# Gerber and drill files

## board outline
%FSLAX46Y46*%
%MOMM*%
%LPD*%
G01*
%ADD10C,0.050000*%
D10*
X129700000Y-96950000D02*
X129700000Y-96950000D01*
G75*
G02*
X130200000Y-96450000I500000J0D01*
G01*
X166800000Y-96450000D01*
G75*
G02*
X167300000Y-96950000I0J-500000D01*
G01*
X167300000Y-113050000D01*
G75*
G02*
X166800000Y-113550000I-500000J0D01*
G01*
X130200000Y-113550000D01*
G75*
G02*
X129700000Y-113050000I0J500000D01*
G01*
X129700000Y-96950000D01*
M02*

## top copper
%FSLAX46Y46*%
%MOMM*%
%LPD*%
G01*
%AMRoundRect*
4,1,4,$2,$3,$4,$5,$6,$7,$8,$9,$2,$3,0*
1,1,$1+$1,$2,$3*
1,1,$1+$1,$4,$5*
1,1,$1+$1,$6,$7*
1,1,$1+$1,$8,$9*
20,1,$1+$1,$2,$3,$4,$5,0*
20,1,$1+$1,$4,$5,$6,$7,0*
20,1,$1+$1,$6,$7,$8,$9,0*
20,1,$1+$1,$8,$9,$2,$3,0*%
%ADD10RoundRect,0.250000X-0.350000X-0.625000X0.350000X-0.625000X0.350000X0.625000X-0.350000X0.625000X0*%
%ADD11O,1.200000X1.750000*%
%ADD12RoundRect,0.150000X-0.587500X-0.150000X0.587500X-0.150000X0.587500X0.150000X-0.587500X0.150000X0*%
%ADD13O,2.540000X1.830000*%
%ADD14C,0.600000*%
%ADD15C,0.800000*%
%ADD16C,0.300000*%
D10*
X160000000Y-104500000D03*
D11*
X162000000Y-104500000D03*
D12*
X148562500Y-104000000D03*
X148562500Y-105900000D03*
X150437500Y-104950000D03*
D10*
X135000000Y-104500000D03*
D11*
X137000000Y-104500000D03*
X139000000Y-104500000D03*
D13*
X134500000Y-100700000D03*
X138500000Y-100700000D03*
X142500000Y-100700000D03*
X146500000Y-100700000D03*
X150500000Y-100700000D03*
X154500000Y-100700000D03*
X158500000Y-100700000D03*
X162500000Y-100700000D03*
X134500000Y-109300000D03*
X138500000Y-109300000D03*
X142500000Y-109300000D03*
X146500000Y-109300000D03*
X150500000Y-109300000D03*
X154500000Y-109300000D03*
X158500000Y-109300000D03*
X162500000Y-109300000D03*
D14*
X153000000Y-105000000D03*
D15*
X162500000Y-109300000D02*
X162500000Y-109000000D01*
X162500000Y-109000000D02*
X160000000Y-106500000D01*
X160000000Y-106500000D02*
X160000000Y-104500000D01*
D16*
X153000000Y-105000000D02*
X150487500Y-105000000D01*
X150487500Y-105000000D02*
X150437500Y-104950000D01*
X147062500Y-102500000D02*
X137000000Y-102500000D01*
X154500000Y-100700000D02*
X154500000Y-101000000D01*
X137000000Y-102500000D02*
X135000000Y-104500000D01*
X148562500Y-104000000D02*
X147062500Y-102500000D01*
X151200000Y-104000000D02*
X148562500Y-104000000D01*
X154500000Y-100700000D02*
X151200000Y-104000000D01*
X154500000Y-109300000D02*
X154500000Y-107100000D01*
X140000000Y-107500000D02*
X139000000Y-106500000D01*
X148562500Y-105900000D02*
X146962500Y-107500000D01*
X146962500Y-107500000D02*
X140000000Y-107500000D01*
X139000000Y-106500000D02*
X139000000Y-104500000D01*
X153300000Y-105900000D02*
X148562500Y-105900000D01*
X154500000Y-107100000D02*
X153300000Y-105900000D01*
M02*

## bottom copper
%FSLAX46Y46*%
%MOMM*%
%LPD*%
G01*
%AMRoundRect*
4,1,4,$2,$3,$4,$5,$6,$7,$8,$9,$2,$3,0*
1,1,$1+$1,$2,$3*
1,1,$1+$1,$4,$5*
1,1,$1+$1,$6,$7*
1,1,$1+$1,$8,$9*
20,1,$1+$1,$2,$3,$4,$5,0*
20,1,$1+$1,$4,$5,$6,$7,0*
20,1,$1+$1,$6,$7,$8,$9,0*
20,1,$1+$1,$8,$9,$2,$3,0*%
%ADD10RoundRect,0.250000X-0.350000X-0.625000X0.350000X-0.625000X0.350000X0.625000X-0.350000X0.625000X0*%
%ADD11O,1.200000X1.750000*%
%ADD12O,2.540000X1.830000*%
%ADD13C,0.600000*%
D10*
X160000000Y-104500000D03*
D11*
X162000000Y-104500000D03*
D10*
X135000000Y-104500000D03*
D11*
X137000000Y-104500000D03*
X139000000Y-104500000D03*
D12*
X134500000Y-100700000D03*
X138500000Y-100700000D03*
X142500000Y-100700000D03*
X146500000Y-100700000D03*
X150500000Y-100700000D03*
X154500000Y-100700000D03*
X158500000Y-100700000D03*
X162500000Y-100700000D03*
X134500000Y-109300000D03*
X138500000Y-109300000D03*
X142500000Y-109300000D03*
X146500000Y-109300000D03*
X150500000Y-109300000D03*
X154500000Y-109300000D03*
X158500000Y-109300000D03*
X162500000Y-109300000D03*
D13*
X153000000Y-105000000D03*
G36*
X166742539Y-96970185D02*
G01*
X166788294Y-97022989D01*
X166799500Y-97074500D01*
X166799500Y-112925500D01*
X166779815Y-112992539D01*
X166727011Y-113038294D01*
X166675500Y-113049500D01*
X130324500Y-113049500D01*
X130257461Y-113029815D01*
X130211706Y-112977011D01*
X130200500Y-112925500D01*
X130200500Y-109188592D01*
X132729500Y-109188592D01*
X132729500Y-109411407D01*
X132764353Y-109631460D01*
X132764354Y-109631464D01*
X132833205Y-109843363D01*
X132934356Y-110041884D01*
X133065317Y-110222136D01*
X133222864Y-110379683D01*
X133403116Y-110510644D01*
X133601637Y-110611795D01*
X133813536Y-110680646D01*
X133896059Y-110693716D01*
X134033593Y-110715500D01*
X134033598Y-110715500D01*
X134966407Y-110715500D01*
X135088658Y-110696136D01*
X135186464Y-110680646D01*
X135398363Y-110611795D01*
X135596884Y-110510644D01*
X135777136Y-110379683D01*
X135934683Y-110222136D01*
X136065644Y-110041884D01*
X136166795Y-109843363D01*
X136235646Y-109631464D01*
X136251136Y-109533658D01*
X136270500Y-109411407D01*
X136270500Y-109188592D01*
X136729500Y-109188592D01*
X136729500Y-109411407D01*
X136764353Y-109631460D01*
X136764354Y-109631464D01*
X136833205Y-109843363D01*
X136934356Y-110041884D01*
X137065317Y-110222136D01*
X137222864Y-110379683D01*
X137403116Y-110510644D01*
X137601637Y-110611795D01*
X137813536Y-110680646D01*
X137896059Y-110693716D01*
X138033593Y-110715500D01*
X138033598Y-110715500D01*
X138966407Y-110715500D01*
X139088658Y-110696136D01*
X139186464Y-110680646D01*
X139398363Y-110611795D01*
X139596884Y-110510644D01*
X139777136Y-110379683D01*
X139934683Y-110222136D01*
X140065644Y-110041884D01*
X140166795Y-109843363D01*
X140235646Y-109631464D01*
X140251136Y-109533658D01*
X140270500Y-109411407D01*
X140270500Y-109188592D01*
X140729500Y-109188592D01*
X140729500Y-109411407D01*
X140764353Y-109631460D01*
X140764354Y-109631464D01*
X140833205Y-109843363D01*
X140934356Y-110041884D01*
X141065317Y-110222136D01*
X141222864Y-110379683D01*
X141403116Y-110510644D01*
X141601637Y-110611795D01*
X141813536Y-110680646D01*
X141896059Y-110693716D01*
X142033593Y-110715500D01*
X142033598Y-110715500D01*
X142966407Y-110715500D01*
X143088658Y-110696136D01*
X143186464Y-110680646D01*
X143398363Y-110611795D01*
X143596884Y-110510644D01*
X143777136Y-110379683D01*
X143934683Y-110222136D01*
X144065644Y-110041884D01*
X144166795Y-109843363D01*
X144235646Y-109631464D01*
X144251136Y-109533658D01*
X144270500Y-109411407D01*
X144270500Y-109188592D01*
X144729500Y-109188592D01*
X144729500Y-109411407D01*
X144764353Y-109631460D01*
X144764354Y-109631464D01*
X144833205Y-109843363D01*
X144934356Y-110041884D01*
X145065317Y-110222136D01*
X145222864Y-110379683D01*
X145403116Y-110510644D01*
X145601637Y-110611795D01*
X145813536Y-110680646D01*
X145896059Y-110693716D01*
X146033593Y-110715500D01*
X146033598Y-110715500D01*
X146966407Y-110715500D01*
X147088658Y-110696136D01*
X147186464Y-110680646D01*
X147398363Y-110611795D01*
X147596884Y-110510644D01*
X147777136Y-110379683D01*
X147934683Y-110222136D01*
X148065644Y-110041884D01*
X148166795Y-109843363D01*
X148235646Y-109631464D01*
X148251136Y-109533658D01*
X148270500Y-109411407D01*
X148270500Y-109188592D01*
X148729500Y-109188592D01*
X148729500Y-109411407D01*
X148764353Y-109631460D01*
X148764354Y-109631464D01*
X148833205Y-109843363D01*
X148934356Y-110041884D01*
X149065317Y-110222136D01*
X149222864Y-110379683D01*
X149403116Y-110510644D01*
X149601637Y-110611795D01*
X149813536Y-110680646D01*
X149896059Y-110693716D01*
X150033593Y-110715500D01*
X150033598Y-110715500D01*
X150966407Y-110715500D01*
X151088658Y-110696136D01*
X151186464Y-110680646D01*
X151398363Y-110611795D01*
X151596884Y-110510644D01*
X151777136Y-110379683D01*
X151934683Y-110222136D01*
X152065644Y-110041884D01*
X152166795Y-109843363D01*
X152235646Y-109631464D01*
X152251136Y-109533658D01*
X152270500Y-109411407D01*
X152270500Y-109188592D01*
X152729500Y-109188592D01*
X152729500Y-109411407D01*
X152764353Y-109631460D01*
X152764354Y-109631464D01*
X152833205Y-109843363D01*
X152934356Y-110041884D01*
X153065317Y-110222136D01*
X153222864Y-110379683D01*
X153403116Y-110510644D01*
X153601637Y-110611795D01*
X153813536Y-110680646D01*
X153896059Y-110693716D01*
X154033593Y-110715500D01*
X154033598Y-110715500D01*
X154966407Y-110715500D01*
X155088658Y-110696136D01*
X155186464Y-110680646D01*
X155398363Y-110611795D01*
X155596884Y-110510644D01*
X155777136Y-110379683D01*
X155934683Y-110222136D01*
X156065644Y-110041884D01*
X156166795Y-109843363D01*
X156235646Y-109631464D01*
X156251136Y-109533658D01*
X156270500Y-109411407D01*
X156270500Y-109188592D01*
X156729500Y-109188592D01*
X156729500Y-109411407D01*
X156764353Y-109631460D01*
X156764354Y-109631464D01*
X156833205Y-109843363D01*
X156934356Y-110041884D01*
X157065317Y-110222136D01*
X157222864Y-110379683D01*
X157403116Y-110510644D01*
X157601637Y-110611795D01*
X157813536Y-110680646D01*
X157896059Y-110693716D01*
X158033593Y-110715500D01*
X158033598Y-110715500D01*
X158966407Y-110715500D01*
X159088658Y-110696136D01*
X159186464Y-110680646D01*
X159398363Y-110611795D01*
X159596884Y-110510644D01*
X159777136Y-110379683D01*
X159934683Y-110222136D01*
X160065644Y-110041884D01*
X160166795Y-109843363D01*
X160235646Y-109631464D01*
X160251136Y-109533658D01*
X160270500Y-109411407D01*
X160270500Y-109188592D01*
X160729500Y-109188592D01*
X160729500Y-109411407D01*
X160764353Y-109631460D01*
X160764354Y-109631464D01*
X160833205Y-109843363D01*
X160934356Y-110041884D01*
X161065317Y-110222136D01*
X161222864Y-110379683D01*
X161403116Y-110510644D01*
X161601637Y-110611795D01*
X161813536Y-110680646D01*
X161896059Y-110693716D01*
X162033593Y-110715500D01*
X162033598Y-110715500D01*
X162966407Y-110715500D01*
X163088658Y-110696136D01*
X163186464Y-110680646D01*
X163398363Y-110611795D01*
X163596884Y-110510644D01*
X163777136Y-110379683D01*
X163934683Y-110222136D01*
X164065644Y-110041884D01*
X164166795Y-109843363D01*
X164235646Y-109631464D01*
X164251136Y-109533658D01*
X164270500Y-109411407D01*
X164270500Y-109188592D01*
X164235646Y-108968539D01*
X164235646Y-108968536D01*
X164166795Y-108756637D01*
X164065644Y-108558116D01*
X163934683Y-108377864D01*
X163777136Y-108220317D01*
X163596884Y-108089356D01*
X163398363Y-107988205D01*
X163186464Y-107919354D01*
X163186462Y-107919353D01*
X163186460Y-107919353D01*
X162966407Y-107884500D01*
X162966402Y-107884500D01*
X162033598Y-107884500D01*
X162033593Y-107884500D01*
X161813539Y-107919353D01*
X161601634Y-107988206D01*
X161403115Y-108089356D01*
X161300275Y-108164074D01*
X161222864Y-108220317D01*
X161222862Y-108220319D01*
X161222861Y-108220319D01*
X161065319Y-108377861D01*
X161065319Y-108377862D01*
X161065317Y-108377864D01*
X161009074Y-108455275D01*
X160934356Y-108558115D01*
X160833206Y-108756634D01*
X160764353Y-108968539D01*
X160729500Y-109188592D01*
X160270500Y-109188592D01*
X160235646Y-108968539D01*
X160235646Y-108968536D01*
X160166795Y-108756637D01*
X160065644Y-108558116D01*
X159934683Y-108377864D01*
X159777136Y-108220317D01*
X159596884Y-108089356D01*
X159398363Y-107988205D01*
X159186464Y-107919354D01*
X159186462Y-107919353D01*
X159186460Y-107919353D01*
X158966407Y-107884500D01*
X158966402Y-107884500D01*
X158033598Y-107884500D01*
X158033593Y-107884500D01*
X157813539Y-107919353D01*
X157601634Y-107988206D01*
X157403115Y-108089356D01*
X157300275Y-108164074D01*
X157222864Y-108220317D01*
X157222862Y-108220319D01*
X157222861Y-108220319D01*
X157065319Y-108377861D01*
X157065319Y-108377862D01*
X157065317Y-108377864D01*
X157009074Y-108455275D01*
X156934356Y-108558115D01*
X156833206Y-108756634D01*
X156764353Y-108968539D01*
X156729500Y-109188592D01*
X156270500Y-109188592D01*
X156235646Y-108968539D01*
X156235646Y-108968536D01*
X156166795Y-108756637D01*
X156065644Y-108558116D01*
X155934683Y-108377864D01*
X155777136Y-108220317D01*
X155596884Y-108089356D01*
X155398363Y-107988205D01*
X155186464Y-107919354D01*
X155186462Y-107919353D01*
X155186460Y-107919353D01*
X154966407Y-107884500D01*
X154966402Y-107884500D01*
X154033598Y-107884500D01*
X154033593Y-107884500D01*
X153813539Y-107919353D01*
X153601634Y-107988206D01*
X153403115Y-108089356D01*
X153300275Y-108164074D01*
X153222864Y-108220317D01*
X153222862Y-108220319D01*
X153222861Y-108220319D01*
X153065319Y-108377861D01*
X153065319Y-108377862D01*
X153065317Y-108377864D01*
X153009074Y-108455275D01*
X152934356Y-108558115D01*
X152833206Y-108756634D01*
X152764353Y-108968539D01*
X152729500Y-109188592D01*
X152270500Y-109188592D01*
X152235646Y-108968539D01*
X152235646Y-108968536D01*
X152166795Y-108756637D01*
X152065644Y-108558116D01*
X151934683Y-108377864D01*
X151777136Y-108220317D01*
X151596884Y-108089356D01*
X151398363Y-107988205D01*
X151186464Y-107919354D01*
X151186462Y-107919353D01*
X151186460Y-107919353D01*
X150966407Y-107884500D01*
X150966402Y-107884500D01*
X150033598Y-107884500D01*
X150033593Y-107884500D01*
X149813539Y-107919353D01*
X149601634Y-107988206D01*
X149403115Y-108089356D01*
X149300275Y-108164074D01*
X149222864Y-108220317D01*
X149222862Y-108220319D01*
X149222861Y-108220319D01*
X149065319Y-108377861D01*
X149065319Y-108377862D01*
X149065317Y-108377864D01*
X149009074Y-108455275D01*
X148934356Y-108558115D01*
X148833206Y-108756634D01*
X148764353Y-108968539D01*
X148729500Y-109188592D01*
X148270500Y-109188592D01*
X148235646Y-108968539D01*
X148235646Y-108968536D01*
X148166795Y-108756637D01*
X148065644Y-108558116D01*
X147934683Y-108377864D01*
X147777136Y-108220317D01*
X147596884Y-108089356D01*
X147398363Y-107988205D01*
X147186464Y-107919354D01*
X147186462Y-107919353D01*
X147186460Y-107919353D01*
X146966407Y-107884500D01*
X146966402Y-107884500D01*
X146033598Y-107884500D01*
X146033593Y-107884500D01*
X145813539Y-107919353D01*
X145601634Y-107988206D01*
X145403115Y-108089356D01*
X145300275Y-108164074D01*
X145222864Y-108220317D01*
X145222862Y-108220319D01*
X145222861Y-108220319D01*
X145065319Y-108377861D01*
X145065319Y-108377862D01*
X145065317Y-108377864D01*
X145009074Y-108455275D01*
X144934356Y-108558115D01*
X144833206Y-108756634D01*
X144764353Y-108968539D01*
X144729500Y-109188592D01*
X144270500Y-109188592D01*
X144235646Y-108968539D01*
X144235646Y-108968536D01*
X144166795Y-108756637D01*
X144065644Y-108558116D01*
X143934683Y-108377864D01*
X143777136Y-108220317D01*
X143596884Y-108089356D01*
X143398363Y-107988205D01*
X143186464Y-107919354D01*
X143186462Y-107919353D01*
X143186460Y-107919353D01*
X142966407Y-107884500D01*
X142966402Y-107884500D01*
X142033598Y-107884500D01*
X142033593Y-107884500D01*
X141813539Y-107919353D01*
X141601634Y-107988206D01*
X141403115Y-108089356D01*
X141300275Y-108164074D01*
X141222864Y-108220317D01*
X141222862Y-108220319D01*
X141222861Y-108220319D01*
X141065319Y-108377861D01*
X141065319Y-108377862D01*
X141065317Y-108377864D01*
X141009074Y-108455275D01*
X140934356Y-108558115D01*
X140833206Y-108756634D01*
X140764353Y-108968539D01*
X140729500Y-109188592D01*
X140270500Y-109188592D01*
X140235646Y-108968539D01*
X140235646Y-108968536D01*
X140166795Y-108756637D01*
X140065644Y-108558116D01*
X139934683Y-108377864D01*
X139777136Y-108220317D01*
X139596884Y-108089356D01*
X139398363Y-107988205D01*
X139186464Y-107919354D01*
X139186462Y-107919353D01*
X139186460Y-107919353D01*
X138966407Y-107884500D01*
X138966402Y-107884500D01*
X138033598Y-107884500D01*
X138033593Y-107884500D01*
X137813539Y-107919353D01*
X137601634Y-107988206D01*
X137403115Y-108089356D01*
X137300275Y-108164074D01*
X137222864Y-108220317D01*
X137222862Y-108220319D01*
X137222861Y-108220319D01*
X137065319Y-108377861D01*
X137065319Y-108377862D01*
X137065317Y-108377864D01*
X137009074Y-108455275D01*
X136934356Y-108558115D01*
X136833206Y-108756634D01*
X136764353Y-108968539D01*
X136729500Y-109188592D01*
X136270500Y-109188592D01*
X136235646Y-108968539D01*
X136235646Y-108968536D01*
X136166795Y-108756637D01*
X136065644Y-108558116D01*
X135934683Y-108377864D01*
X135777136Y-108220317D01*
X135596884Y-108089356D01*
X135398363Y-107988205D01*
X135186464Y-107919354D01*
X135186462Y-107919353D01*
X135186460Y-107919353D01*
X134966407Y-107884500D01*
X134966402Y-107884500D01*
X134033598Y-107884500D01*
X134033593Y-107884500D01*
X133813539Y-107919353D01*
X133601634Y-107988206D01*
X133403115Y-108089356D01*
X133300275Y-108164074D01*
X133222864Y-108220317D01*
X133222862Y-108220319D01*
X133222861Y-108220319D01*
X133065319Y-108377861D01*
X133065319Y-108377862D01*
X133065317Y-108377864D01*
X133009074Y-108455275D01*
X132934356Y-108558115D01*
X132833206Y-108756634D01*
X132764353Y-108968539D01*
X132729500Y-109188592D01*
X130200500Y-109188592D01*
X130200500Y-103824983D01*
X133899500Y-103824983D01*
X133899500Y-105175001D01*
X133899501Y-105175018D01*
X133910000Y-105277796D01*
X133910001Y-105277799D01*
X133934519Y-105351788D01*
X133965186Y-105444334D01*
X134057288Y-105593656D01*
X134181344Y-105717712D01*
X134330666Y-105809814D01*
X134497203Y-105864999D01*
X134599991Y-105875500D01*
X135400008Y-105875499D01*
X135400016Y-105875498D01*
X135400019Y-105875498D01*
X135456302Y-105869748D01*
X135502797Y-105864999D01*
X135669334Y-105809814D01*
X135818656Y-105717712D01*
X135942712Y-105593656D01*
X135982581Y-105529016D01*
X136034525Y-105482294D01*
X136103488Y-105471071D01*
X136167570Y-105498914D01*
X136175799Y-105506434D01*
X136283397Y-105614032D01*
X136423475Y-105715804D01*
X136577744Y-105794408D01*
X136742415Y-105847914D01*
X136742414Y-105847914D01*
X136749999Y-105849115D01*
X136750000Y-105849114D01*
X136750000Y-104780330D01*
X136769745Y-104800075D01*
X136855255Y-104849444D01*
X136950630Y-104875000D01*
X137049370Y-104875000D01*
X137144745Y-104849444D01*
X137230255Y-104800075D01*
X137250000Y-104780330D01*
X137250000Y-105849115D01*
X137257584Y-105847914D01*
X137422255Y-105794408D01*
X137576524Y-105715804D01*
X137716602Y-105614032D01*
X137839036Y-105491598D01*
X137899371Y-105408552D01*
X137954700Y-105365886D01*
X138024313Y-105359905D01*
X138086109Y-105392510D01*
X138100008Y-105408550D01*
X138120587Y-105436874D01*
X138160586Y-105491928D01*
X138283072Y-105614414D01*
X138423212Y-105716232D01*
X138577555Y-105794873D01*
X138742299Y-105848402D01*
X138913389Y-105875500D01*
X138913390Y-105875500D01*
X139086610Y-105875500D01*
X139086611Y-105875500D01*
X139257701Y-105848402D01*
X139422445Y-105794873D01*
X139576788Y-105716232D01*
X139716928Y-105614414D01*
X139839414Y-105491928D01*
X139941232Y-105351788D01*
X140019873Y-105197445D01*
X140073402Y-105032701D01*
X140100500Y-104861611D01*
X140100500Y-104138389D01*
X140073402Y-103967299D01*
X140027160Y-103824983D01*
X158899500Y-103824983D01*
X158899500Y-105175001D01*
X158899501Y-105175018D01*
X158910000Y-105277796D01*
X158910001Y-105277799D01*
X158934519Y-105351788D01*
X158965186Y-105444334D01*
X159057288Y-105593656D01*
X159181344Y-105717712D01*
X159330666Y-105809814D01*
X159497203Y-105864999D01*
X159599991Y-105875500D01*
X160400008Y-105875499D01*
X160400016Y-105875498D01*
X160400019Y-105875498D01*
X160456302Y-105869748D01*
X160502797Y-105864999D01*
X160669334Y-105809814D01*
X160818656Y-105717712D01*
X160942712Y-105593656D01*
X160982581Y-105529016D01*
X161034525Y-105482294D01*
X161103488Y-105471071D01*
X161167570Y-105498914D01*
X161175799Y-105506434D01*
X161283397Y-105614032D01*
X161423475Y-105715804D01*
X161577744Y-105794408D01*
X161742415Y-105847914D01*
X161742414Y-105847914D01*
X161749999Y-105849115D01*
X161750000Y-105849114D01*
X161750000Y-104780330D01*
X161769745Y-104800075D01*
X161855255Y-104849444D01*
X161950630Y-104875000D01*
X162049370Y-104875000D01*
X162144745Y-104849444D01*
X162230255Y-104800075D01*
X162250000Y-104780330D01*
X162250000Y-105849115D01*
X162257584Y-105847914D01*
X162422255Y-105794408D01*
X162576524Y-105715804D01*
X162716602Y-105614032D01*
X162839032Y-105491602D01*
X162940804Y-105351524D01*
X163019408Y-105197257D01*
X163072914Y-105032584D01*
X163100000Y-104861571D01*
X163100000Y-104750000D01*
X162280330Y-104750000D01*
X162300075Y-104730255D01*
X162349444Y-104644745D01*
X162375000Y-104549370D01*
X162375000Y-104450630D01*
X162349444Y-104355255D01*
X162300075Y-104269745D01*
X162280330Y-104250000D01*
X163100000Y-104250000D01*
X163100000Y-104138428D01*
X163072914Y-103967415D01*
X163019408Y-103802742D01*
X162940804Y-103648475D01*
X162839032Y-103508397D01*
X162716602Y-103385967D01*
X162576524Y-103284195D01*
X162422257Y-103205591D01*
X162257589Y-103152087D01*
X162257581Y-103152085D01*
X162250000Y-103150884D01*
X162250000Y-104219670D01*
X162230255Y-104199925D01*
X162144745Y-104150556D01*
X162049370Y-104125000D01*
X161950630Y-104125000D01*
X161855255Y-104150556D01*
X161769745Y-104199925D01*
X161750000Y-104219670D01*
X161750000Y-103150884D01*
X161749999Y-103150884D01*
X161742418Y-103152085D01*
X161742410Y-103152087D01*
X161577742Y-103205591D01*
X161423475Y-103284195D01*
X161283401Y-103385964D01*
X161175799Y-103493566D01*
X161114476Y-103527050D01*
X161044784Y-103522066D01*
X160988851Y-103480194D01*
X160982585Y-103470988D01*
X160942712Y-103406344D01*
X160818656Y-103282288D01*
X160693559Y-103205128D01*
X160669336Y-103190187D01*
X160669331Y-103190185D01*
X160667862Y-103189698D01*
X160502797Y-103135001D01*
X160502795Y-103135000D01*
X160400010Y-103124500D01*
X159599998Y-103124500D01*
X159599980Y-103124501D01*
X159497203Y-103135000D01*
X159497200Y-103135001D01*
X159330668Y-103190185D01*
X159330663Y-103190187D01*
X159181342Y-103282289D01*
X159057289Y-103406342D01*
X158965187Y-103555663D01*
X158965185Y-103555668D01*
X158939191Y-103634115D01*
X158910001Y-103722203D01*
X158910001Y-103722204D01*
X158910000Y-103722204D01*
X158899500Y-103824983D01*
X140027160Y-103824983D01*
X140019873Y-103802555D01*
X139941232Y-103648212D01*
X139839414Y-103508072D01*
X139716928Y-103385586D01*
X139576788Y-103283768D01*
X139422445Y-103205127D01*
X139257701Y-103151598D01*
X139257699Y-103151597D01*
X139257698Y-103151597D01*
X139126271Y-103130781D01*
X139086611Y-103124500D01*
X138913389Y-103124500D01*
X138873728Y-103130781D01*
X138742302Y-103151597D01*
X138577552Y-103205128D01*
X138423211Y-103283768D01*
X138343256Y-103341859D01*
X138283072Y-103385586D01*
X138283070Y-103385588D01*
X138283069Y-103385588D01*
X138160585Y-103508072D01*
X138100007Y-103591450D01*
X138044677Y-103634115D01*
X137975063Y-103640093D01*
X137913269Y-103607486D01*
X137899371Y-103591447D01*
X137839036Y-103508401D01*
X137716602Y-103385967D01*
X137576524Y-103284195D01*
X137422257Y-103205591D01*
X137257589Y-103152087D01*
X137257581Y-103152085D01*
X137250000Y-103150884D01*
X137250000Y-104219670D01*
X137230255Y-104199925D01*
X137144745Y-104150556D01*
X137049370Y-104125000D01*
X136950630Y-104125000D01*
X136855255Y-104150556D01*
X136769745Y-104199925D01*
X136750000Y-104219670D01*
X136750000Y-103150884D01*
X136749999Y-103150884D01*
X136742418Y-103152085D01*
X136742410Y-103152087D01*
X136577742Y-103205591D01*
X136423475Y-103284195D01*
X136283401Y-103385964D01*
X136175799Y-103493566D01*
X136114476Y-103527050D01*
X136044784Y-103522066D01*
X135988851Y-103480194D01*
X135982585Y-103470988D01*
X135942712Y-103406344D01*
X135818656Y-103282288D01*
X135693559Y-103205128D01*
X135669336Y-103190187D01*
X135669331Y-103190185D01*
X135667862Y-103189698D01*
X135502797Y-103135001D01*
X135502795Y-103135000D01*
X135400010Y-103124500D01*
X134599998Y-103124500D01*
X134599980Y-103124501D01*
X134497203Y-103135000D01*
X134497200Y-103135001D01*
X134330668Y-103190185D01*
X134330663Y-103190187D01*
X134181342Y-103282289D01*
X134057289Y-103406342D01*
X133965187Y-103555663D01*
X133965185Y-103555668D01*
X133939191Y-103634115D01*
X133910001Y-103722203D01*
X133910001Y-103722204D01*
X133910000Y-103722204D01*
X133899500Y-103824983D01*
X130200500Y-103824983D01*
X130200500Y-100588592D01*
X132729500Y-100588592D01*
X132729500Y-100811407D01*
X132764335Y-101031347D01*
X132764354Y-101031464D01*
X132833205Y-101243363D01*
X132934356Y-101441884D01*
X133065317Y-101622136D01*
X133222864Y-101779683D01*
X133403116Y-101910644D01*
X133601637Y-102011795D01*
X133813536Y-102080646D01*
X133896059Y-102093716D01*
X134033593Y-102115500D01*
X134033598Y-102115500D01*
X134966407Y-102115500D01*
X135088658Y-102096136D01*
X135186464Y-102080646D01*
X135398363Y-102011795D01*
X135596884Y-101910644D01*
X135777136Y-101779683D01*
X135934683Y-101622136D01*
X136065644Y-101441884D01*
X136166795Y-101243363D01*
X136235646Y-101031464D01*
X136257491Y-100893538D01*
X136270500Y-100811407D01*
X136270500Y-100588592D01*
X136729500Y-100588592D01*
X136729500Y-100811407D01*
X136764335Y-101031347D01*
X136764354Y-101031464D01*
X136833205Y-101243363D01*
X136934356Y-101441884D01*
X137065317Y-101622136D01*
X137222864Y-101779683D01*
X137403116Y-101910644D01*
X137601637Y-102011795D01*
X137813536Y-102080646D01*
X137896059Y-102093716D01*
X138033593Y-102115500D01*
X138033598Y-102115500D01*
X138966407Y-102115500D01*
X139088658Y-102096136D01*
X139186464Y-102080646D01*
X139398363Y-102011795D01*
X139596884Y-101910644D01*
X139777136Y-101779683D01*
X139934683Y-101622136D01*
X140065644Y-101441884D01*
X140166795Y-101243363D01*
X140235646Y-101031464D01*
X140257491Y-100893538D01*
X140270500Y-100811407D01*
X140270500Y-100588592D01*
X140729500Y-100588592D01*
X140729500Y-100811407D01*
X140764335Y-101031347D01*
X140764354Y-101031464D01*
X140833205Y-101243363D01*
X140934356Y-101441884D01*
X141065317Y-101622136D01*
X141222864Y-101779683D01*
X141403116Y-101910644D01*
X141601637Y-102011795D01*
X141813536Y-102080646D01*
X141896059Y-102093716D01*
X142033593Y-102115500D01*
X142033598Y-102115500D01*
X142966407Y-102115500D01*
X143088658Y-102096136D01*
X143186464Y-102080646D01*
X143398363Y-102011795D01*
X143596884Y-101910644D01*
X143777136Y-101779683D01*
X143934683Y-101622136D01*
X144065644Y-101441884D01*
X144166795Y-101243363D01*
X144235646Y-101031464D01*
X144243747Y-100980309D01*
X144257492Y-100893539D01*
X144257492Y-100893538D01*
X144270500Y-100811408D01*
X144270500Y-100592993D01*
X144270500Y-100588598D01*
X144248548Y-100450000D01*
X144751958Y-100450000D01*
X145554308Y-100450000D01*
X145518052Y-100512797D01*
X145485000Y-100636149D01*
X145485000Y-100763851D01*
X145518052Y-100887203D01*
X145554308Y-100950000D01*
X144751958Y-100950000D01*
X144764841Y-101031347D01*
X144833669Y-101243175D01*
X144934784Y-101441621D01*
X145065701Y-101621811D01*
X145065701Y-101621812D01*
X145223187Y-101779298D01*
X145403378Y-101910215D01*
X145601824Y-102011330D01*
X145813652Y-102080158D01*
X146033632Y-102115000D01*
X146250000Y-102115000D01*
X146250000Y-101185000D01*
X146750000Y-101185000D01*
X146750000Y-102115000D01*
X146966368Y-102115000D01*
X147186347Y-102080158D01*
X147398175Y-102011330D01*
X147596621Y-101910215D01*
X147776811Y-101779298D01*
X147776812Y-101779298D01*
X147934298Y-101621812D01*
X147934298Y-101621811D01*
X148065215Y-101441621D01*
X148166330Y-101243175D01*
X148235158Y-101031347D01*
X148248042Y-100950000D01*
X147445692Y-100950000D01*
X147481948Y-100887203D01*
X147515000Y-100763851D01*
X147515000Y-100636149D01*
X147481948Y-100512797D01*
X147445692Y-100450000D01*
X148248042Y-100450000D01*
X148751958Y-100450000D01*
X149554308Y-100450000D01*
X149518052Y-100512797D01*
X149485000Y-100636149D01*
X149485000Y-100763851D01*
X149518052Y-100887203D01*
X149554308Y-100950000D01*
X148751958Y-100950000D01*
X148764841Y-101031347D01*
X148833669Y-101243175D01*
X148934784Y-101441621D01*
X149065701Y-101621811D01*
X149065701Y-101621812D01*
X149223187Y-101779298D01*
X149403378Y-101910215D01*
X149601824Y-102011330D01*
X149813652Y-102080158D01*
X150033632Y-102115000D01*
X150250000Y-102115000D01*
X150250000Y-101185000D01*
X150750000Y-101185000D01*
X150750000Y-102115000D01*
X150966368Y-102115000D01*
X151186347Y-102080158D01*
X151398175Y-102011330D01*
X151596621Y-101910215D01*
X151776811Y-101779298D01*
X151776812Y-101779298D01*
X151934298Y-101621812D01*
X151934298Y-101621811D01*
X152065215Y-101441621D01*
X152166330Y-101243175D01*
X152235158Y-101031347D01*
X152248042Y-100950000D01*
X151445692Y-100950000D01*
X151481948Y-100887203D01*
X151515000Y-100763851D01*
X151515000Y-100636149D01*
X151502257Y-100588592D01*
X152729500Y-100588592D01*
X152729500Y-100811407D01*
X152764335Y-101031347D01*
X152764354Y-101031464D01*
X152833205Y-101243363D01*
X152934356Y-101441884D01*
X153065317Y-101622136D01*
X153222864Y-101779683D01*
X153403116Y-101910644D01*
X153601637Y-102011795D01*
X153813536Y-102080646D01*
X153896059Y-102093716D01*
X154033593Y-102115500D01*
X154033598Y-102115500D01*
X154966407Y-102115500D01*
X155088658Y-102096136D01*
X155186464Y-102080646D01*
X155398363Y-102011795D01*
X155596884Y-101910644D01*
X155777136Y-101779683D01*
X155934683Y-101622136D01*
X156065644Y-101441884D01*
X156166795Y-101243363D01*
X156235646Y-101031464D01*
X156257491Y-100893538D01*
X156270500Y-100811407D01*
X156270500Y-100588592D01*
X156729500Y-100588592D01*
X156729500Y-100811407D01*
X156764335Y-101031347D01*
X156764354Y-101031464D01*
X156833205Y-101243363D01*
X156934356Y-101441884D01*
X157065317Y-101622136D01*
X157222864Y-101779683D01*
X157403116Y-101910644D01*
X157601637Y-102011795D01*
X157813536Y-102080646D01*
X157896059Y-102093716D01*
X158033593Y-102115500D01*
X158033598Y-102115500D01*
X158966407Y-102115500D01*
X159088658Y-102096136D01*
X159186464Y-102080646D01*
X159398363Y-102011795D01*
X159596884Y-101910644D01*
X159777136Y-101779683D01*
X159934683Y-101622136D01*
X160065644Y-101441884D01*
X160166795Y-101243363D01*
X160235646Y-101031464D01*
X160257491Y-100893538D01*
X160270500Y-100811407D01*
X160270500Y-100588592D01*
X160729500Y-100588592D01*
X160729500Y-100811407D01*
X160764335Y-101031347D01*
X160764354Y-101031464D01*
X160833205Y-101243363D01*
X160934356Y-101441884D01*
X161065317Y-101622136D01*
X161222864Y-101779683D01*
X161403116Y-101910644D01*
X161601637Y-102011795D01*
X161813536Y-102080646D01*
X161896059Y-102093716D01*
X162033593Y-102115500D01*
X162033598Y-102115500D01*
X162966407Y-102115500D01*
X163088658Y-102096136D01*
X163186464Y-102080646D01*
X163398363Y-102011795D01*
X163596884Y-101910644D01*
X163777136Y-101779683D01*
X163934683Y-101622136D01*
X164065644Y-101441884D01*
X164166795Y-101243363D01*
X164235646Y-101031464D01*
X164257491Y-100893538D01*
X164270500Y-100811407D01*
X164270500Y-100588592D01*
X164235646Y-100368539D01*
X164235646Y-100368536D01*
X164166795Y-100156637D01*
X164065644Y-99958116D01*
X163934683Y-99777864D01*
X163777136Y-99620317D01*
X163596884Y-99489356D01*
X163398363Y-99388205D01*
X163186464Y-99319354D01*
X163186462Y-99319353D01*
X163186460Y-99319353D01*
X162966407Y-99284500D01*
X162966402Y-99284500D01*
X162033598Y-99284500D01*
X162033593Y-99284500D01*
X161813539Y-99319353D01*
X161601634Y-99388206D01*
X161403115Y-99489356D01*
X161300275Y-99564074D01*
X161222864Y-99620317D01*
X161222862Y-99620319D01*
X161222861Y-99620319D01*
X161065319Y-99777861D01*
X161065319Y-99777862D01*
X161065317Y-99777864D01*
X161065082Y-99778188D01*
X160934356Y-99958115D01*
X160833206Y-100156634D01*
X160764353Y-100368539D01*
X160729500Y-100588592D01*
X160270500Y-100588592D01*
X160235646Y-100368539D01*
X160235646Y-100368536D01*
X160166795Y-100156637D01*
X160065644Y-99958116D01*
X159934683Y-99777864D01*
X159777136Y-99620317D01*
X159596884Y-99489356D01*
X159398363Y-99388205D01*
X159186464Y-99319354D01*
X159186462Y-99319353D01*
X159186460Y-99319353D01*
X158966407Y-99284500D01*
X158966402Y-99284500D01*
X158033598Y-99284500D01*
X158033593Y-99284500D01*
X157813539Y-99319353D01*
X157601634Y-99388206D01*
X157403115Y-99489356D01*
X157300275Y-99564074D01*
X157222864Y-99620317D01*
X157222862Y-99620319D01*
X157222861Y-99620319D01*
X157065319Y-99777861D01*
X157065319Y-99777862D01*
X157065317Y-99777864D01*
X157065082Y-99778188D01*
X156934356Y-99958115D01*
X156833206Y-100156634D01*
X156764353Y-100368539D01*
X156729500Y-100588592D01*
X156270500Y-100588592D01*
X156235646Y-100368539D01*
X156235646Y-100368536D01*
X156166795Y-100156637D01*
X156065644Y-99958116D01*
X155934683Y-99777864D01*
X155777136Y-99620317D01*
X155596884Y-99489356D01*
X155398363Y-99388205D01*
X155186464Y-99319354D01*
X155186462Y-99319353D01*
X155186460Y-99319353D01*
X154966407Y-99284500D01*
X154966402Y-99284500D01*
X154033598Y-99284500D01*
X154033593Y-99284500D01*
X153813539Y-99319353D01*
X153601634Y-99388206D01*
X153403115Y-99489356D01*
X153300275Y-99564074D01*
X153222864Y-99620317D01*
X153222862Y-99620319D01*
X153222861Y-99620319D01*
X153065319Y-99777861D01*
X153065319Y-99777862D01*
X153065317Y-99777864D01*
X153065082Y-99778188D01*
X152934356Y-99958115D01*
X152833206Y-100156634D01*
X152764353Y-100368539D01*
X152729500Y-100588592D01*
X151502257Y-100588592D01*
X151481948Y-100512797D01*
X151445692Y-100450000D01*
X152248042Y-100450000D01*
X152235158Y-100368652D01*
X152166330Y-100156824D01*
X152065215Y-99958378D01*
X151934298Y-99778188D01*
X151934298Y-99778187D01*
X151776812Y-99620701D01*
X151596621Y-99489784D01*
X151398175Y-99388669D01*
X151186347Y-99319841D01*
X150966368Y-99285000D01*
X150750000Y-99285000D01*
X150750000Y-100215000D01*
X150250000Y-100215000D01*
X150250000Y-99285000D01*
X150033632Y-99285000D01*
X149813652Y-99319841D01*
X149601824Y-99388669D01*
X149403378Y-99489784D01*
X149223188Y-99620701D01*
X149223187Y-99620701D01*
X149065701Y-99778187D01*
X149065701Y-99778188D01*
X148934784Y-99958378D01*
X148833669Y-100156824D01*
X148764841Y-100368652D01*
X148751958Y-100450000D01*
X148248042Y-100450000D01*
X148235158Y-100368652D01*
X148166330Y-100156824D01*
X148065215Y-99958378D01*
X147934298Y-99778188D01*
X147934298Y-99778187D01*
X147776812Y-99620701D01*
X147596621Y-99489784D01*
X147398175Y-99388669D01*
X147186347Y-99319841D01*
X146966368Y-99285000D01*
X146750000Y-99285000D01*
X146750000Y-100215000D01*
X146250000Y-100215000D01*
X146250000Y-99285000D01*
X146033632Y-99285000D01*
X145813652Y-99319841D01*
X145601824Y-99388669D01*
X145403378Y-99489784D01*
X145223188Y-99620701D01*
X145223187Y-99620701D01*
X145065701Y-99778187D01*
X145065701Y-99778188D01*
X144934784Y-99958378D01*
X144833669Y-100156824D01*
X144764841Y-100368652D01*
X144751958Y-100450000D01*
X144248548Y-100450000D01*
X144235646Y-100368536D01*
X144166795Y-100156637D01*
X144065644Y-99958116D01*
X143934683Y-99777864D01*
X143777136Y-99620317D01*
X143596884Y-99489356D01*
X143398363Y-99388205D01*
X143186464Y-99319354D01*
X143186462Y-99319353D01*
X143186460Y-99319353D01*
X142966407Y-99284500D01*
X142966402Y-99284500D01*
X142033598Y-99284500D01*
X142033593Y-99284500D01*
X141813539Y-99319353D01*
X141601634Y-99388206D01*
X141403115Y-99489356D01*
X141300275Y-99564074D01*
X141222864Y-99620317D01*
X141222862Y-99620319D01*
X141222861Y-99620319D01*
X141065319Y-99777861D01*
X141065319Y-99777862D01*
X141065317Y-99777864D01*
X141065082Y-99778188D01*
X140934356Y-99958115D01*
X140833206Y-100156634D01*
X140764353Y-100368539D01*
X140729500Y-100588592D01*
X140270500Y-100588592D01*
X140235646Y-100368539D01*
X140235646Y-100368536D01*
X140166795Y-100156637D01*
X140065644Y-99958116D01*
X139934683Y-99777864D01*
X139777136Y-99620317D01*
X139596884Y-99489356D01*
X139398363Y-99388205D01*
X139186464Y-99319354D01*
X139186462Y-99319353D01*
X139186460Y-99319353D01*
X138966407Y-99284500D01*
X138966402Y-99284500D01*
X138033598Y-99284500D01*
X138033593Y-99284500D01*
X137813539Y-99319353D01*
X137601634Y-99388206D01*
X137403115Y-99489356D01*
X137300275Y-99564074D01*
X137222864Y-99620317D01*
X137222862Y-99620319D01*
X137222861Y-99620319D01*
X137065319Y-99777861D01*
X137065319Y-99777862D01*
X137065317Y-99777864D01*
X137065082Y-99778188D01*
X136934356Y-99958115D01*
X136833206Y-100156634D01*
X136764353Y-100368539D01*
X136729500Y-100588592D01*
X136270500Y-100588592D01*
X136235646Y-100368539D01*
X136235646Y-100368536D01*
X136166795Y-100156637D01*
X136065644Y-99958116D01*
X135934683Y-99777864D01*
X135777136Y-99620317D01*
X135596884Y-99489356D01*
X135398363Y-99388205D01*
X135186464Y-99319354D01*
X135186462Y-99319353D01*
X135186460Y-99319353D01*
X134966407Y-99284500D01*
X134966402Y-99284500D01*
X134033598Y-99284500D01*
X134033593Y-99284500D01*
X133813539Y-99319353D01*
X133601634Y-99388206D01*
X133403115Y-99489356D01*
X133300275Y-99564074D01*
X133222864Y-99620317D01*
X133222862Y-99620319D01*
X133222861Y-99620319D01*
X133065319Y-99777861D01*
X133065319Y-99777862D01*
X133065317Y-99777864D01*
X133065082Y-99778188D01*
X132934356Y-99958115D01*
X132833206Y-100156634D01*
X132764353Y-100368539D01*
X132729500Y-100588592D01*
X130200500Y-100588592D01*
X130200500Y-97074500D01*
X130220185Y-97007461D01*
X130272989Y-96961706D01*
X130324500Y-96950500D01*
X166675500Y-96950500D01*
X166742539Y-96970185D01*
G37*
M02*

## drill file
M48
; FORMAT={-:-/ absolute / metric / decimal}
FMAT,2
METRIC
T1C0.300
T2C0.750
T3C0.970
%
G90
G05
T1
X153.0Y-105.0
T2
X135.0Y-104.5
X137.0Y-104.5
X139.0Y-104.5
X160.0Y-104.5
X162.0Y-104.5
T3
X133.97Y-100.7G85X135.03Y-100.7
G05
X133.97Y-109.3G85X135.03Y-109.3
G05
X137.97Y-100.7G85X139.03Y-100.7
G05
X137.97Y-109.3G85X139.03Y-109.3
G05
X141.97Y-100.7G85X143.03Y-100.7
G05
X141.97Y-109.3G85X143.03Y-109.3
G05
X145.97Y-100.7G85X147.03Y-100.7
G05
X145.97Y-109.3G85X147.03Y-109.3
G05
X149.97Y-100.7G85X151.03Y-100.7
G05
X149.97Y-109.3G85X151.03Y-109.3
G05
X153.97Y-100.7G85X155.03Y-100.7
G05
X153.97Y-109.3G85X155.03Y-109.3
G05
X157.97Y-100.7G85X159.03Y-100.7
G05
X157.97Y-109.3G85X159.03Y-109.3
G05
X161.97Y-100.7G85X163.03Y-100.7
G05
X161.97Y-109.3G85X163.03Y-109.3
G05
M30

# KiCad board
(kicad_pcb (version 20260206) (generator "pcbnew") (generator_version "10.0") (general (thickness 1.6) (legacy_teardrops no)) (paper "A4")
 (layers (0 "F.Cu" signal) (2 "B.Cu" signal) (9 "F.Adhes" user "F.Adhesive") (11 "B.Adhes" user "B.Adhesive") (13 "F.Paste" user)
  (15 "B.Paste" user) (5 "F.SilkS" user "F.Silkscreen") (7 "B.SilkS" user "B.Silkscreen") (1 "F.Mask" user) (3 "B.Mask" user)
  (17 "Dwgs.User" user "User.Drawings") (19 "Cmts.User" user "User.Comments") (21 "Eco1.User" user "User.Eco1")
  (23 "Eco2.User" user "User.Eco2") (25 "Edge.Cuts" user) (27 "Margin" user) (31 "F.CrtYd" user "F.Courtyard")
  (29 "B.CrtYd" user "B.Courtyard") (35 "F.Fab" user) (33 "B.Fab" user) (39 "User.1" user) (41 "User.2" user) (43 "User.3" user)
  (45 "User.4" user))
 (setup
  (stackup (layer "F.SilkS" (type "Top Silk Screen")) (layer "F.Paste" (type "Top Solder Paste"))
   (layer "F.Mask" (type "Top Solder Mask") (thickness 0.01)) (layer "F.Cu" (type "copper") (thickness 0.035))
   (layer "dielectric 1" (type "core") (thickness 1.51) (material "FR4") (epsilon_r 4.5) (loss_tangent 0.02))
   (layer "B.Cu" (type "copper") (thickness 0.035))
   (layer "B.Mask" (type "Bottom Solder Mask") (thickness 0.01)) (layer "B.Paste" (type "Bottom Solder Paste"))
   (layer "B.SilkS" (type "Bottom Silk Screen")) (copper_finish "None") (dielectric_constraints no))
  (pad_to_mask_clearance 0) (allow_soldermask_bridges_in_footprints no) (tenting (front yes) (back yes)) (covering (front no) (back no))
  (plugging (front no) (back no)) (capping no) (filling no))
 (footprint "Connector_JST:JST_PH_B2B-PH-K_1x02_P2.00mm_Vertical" (layer "F.Cu") (at 160 104.5)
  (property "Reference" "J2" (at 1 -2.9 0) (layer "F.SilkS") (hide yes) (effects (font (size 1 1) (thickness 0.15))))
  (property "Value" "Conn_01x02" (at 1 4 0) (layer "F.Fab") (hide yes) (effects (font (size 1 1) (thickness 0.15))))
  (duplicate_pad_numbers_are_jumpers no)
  (pad "1" thru_hole roundrect (at 0 0) (size 1.2 1.75) (drill 0.75) (layers "*.Cu" "*.Mask") (remove_unused_layers no)
   (roundrect_rratio 0.208333) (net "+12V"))
  (pad "2" thru_hole oval (at 2 0) (size 1.2 1.75) (drill 0.75) (layers "*.Cu" "*.Mask") (remove_unused_layers no) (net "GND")))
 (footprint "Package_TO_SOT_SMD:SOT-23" (layer "F.Cu") (at 149.5 104.95)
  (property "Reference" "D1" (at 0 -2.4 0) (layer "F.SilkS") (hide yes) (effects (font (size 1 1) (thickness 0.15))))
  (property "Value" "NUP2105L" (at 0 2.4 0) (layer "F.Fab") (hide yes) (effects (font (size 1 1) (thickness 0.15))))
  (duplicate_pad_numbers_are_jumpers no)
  (pad "1" smd roundrect (at -0.9375 -0.95) (size 1.475 0.6) (layers "F.Cu" "F.Mask" "F.Paste") (roundrect_rratio 0.25) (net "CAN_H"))
  (pad "2" smd roundrect (at -0.9375 0.95) (size 1.475 0.6) (layers "F.Cu" "F.Mask" "F.Paste") (roundrect_rratio 0.25) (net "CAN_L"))
  (pad "3" smd roundrect (at 0.9375 0) (size 1.475 0.6) (layers "F.Cu" "F.Mask" "F.Paste") (roundrect_rratio 0.25) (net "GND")))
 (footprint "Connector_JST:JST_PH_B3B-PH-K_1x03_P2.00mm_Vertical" (layer "F.Cu") (at 135 104.5)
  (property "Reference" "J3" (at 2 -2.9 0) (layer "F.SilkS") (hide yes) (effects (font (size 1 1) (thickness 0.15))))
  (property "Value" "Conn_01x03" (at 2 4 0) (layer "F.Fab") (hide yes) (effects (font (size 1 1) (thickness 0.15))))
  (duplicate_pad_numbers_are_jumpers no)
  (pad "1" thru_hole roundrect (at 0 0) (size 1.2 1.75) (drill 0.75) (layers "*.Cu" "*.Mask") (remove_unused_layers no)
   (roundrect_rratio 0.208333) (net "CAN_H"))
  (pad "2" thru_hole oval (at 2 0) (size 1.2 1.75) (drill 0.75) (layers "*.Cu" "*.Mask") (remove_unused_layers no) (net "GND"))
  (pad "3" thru_hole oval (at 4 0) (size 1.2 1.75) (drill 0.75) (layers "*.Cu" "*.Mask") (remove_unused_layers no) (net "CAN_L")))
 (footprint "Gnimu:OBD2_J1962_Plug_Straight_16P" (layer "F.Cu") (at 148.5 105)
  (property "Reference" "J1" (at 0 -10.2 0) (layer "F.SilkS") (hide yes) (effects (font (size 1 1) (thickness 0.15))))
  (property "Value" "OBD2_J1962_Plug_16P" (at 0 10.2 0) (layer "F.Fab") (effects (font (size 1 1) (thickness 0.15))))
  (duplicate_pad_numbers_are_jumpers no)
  (pad "1" thru_hole oval (at -14 -4.3) (size 2.54 1.83) (drill oval 2.03 0.97) (layers "*.Cu" "*.Mask") (remove_unused_layers no)
   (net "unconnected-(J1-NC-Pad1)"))
  (pad "2" thru_hole oval (at -10 -4.3) (size 2.54 1.83) (drill oval 2.03 0.97) (layers "*.Cu" "*.Mask") (remove_unused_layers no)
   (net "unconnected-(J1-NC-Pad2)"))
  (pad "3" thru_hole oval (at -6 -4.3) (size 2.54 1.83) (drill oval 2.03 0.97) (layers "*.Cu" "*.Mask") (remove_unused_layers no)
   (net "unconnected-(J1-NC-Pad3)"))
  (pad "4" thru_hole oval (at -2 -4.3) (size 2.54 1.83) (drill oval 2.03 0.97) (layers "*.Cu" "*.Mask") (remove_unused_layers no)
   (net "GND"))
  (pad "5" thru_hole oval (at 2 -4.3) (size 2.54 1.83) (drill oval 2.03 0.97) (layers "*.Cu" "*.Mask") (remove_unused_layers no) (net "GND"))
  (pad "6" thru_hole oval (at 6 -4.3) (size 2.54 1.83) (drill oval 2.03 0.97) (layers "*.Cu" "*.Mask") (remove_unused_layers no)
   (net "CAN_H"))
  (pad "7" thru_hole oval (at 10 -4.3) (size 2.54 1.83) (drill oval 2.03 0.97) (layers "*.Cu" "*.Mask") (remove_unused_layers no)
   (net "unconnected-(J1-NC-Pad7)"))
  (pad "8" thru_hole oval (at 14 -4.3) (size 2.54 1.83) (drill oval 2.03 0.97) (layers "*.Cu" "*.Mask") (remove_unused_layers no)
   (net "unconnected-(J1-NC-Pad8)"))
  (pad "9" thru_hole oval (at -14 4.3) (size 2.54 1.83) (drill oval 2.03 0.97) (layers "*.Cu" "*.Mask") (remove_unused_layers no)
   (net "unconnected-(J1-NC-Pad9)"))
  (pad "10" thru_hole oval (at -10 4.3) (size 2.54 1.83) (drill oval 2.03 0.97) (layers "*.Cu" "*.Mask") (remove_unused_layers no)
   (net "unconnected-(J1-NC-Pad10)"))
  (pad "11" thru_hole oval (at -6 4.3) (size 2.54 1.83) (drill oval 2.03 0.97) (layers "*.Cu" "*.Mask") (remove_unused_layers no)
   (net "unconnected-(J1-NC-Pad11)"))
  (pad "12" thru_hole oval (at -2 4.3) (size 2.54 1.83) (drill oval 2.03 0.97) (layers "*.Cu" "*.Mask") (remove_unused_layers no)
   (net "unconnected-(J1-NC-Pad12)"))
  (pad "13" thru_hole oval (at 2 4.3) (size 2.54 1.83) (drill oval 2.03 0.97) (layers "*.Cu" "*.Mask") (remove_unused_layers no)
   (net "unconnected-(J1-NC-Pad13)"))
  (pad "14" thru_hole oval (at 6 4.3) (size 2.54 1.83) (drill oval 2.03 0.97) (layers "*.Cu" "*.Mask") (remove_unused_layers no)
   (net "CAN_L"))
  (pad "15" thru_hole oval (at 10 4.3) (size 2.54 1.83) (drill oval 2.03 0.97) (layers "*.Cu" "*.Mask") (remove_unused_layers no)
   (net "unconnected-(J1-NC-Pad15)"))
  (pad "16" thru_hole oval (at 14 4.3) (size 2.54 1.83) (drill oval 2.03 0.97) (layers "*.Cu" "*.Mask") (remove_unused_layers no)
   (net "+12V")))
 (gr_rect (start 129.7 96.45) (end 167.3 113.55) (radius 0.5) (stroke (width 0.05) (type solid)) (fill no) (locked yes) (layer "Edge.Cuts"))
 (segment (start 162.5 109.3) (end 162.5 109) (width 0.8) (layer "F.Cu") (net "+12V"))
 (segment (start 162.5 109) (end 160 106.5) (width 0.8) (layer "F.Cu") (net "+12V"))
 (segment (start 160 106.5) (end 160 104.5) (width 0.8) (layer "F.Cu") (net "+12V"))
 (segment (start 153 105) (end 150.4875 105) (width 0.3) (layer "F.Cu") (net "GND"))
 (segment (start 150.4875 105) (end 150.4375 104.95) (width 0.3) (layer "F.Cu") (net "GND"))
 (via (at 153 105) (size 0.6) (drill 0.3) (layers "F.Cu" "B.Cu") (free yes) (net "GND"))
 (segment (start 147.0625 102.5) (end 137 102.5) (width 0.3) (layer "F.Cu") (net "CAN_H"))
 (segment (start 154.5 100.7) (end 154.5 101) (width 0.3) (layer "F.Cu") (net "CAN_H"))
 (segment (start 137 102.5) (end 135 104.5) (width 0.3) (layer "F.Cu") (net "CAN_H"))
 (segment (start 148.5625 104) (end 147.0625 102.5) (width 0.3) (layer "F.Cu") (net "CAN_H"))
 (segment (start 151.2 104) (end 148.5625 104) (width 0.3) (layer "F.Cu") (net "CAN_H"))
 (segment (start 154.5 100.7) (end 151.2 104) (width 0.3) (layer "F.Cu") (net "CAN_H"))
 (segment (start 154.5 109.3) (end 154.5 107.1) (width 0.3) (layer "F.Cu") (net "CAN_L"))
 (segment (start 140 107.5) (end 139 106.5) (width 0.3) (layer "F.Cu") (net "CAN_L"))
 (segment (start 148.5625 105.9) (end 146.9625 107.5) (width 0.3) (layer "F.Cu") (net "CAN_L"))
 (segment (start 146.9625 107.5) (end 140 107.5) (width 0.3) (layer "F.Cu") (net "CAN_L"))
 (segment (start 139 106.5) (end 139 104.5) (width 0.3) (layer "F.Cu") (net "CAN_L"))
 (segment (start 153.3 105.9) (end 148.5625 105.9) (width 0.3) (layer "F.Cu") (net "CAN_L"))
 (segment (start 154.5 107.1) (end 153.3 105.9) (width 0.3) (layer "F.Cu") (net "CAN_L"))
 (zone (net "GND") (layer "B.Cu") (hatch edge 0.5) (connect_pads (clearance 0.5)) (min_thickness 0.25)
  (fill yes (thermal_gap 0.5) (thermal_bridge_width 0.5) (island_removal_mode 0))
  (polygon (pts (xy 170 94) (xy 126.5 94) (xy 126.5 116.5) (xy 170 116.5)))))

